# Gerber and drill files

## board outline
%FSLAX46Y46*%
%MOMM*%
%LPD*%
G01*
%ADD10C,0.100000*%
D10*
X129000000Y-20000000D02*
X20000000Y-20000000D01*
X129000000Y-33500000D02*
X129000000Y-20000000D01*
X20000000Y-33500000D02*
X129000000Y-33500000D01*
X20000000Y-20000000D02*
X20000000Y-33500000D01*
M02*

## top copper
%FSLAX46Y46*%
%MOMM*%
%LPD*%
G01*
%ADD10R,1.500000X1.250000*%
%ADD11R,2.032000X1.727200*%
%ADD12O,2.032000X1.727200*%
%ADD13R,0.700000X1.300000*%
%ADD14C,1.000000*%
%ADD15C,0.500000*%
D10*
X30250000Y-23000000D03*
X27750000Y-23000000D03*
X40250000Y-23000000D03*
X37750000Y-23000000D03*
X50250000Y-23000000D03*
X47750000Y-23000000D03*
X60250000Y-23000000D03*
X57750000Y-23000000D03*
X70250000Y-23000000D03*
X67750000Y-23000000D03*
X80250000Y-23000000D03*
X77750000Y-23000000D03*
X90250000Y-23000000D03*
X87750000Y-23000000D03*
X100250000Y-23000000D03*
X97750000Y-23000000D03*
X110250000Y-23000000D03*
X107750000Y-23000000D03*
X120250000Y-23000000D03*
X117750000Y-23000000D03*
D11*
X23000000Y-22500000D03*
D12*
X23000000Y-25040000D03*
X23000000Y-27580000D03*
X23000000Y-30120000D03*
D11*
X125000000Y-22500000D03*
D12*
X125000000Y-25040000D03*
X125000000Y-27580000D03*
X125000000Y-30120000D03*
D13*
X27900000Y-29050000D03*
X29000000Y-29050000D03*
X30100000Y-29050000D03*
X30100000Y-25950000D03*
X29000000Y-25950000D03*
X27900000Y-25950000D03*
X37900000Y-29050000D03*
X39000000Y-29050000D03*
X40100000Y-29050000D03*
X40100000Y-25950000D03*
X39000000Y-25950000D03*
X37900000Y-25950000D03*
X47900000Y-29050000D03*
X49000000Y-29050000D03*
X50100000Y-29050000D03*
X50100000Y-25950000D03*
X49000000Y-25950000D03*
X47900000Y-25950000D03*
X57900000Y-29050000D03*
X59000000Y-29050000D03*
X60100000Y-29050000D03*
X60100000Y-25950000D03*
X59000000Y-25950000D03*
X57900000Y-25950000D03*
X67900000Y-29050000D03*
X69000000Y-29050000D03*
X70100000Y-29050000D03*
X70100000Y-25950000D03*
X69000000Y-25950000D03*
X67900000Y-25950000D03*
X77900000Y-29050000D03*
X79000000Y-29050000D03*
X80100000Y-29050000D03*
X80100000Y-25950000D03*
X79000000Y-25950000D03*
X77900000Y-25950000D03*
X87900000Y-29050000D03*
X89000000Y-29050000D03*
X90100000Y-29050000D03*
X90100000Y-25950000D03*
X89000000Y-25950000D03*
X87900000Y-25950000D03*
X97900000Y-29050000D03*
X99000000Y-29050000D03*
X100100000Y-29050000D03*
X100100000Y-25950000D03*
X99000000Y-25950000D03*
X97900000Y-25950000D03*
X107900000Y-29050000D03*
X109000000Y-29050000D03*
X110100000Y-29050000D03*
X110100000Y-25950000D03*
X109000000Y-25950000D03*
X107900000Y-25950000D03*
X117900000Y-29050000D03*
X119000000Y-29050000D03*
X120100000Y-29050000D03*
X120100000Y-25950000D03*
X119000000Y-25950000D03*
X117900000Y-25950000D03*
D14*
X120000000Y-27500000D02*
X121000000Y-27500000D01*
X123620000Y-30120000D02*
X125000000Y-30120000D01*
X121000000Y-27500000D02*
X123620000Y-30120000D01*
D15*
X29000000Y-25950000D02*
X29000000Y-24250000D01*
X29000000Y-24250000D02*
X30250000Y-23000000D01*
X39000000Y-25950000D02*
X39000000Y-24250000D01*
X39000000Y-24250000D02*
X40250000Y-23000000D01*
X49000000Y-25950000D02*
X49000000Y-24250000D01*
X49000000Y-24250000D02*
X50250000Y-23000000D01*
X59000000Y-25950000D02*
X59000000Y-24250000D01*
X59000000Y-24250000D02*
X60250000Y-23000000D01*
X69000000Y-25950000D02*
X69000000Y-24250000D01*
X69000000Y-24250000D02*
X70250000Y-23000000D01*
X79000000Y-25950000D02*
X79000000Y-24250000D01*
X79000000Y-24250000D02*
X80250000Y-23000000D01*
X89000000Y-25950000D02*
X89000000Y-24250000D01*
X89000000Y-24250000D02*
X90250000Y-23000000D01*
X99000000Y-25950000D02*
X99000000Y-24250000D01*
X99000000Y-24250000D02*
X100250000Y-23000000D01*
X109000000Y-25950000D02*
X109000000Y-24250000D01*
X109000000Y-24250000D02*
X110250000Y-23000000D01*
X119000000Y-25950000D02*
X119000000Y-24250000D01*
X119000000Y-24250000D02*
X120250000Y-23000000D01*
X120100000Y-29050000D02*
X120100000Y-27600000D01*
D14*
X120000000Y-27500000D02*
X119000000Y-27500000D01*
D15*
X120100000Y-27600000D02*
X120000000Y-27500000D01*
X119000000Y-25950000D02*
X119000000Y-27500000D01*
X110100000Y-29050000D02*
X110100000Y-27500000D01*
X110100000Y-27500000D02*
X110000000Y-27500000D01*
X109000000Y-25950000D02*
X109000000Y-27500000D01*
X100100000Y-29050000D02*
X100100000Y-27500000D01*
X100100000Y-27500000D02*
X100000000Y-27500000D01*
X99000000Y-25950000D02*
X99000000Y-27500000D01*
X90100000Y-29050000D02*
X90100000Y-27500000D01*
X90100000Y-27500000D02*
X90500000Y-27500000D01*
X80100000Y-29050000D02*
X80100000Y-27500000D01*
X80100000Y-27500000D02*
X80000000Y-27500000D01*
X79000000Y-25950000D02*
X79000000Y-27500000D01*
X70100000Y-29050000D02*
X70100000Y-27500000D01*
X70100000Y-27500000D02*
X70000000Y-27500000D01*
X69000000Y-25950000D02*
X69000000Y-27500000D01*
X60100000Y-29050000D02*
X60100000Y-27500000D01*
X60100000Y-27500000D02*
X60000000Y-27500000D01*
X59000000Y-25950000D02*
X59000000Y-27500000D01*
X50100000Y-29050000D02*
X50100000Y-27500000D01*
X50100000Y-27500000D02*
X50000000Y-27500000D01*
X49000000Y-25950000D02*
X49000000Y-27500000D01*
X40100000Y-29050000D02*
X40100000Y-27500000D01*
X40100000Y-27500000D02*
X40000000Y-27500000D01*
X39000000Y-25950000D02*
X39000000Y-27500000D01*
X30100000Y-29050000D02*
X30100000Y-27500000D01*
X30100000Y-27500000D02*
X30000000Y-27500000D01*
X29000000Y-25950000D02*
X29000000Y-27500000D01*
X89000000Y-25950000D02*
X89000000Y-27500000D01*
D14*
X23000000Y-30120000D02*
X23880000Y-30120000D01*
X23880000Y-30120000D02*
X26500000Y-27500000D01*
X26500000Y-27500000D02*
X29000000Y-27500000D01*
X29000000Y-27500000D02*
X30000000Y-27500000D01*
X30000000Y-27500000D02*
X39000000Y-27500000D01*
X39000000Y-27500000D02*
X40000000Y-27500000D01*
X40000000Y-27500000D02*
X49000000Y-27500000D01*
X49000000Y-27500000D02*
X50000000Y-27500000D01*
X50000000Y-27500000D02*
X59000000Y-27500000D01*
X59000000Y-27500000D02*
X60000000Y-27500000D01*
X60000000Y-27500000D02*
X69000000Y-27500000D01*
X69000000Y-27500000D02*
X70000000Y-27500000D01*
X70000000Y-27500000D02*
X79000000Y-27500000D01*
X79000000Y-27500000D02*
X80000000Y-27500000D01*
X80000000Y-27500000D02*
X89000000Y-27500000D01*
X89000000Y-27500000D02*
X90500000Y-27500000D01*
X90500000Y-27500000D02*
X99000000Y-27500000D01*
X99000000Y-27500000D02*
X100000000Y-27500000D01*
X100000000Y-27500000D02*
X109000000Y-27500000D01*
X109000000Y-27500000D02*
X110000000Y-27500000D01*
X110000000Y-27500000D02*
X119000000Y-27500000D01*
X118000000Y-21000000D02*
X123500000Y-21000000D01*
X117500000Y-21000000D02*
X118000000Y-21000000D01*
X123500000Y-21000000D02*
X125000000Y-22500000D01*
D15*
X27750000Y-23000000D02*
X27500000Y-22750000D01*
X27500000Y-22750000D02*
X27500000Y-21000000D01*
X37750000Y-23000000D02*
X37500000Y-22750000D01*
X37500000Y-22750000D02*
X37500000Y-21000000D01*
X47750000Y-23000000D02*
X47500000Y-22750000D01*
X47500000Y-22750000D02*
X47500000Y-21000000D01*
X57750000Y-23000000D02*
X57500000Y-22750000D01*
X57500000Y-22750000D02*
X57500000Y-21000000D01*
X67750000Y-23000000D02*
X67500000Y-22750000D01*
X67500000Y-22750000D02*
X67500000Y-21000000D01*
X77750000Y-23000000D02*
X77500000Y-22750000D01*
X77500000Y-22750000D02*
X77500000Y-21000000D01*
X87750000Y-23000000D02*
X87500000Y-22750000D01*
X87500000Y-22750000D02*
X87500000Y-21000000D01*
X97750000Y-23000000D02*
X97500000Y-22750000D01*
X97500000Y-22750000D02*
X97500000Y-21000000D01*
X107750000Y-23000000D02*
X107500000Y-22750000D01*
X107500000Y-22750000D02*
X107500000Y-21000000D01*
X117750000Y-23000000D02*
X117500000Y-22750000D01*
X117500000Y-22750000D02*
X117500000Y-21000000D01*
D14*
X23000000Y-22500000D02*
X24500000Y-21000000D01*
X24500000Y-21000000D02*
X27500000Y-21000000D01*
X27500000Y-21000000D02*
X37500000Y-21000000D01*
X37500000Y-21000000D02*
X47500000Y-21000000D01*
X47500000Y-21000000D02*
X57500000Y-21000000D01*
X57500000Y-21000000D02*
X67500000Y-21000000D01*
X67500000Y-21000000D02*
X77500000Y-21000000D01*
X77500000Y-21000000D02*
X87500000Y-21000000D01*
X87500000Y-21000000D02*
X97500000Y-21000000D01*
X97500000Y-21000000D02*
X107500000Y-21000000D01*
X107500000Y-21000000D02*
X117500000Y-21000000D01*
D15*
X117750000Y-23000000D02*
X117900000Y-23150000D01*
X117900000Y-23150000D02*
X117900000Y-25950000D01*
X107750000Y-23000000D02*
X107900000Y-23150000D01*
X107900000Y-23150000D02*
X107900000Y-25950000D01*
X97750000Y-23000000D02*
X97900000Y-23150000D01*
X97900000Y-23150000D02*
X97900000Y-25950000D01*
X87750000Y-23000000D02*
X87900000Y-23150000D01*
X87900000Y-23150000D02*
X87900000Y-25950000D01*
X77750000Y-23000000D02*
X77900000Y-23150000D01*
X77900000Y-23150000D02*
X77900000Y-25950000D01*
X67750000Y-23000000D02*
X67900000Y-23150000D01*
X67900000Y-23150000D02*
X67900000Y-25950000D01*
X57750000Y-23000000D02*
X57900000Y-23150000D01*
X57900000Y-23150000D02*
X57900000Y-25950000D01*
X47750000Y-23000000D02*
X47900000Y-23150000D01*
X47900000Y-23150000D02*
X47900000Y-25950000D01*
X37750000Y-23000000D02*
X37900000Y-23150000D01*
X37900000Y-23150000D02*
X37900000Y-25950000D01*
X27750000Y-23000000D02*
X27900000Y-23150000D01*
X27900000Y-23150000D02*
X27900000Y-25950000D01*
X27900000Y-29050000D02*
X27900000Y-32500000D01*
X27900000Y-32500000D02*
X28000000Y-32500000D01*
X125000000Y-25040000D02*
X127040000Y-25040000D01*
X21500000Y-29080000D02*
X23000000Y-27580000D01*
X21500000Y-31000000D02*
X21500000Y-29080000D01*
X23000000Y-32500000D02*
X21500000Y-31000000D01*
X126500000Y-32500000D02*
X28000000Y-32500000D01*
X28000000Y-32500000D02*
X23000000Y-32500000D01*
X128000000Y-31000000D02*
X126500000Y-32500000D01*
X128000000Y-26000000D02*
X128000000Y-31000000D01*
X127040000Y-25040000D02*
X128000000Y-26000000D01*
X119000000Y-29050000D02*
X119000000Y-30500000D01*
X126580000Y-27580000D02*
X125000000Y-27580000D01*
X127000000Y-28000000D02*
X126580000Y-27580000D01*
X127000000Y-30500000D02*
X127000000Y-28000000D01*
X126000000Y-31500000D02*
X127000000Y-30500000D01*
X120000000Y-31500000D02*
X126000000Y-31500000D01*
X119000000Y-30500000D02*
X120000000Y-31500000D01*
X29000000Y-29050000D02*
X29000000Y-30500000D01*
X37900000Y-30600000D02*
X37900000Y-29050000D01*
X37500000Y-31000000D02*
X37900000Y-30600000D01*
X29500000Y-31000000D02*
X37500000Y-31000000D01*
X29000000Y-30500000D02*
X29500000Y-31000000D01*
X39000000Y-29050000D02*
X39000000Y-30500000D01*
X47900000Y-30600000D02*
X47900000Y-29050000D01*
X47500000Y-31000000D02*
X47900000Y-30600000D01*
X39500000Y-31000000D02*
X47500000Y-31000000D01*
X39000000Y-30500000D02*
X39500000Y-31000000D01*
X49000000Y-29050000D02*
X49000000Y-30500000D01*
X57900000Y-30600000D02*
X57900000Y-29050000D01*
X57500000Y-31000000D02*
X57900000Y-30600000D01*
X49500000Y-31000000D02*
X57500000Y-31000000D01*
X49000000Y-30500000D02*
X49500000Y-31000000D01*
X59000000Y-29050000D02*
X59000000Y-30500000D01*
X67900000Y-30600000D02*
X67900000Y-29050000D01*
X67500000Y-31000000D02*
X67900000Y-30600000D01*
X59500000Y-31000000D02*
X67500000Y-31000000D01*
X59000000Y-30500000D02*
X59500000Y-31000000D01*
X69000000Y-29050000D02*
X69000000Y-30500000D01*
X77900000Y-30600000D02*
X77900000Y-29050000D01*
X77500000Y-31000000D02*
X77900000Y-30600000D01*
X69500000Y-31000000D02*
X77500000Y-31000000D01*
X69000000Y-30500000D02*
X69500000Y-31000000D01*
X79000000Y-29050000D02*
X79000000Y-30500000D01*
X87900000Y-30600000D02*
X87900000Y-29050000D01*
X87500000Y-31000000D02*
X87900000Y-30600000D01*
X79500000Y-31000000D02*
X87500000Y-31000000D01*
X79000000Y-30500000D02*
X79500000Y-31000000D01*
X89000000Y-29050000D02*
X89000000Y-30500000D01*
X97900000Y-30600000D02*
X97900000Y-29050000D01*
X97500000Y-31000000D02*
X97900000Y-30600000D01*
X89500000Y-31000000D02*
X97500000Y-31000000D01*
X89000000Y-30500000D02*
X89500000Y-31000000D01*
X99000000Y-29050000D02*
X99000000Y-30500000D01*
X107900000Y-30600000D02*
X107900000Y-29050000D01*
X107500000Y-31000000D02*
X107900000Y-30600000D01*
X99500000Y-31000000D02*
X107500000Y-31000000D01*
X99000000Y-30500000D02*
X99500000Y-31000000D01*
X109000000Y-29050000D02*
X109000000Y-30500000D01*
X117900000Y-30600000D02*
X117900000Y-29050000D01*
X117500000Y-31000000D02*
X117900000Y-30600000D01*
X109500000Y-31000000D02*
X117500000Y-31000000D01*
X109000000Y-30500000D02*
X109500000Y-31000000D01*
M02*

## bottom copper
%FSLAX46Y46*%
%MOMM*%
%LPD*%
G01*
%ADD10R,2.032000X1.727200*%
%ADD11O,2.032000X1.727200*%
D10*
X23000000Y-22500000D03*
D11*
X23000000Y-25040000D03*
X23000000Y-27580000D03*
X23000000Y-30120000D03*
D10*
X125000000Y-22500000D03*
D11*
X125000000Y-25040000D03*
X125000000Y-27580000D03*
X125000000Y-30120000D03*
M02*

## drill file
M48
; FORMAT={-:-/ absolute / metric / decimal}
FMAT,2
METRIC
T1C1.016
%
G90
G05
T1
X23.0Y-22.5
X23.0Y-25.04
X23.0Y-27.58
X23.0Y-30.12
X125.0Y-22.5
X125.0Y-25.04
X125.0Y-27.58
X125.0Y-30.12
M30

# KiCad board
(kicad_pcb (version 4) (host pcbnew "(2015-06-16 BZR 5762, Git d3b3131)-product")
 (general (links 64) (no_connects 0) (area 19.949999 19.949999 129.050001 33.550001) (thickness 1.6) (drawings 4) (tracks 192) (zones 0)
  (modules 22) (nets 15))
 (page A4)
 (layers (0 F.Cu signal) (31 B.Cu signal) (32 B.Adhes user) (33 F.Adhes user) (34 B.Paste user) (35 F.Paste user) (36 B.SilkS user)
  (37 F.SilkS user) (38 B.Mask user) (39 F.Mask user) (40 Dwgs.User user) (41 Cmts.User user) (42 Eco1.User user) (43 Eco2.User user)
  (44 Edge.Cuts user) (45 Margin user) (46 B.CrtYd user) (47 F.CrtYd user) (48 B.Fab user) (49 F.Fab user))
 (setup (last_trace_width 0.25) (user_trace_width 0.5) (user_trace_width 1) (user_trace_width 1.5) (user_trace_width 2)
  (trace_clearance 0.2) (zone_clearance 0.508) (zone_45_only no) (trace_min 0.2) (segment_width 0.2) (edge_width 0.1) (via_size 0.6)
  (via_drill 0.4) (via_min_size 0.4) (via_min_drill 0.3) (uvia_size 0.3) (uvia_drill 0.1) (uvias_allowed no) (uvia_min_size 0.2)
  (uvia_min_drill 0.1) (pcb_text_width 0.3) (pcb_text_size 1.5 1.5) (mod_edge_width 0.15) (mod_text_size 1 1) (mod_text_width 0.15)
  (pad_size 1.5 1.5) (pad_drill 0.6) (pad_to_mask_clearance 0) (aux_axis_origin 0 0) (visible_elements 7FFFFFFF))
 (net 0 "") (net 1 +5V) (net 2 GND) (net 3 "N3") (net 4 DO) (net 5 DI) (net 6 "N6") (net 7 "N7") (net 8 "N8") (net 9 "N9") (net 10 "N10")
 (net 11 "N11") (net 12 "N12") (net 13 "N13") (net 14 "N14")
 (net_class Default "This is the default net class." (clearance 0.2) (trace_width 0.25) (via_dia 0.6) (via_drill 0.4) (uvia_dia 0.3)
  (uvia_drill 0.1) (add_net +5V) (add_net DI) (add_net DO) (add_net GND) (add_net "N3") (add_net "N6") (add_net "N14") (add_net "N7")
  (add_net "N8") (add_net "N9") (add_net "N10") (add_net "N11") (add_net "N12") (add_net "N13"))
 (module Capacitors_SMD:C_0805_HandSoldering (layer F.Cu) (at 29 23 180)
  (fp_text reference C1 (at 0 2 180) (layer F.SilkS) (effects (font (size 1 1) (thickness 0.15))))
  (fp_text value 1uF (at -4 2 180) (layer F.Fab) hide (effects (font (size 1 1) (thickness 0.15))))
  (pad 1 smd rect (at -1.25 0 180) (size 1.5 1.25) (layers F.Cu F.Paste F.Mask) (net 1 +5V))
  (pad 2 smd rect (at 1.25 0 180) (size 1.5 1.25) (layers F.Cu F.Paste F.Mask) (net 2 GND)))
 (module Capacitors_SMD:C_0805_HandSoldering (layer F.Cu) (at 39 23 180)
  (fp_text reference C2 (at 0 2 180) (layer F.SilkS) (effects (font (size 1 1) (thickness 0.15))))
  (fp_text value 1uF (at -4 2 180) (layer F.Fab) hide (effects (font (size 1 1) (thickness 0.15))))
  (pad 1 smd rect (at -1.25 0 180) (size 1.5 1.25) (layers F.Cu F.Paste F.Mask) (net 1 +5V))
  (pad 2 smd rect (at 1.25 0 180) (size 1.5 1.25) (layers F.Cu F.Paste F.Mask) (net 2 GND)))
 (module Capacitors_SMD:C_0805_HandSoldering (layer F.Cu) (at 49 23 180)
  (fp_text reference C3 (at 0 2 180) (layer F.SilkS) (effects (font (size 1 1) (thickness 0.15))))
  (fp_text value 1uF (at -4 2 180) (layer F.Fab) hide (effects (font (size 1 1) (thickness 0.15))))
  (pad 1 smd rect (at -1.25 0 180) (size 1.5 1.25) (layers F.Cu F.Paste F.Mask) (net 1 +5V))
  (pad 2 smd rect (at 1.25 0 180) (size 1.5 1.25) (layers F.Cu F.Paste F.Mask) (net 2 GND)))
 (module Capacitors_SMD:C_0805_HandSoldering (layer F.Cu) (at 59 23 180)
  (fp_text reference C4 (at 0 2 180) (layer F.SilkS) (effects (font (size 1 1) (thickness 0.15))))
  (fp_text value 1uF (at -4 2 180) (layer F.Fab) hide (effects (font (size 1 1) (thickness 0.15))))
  (pad 1 smd rect (at -1.25 0 180) (size 1.5 1.25) (layers F.Cu F.Paste F.Mask) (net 1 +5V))
  (pad 2 smd rect (at 1.25 0 180) (size 1.5 1.25) (layers F.Cu F.Paste F.Mask) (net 2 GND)))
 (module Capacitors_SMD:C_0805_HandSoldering (layer F.Cu) (at 69 23 180)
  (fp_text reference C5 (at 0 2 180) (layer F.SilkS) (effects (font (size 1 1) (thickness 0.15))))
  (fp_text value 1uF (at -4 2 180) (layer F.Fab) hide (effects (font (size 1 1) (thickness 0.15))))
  (pad 1 smd rect (at -1.25 0 180) (size 1.5 1.25) (layers F.Cu F.Paste F.Mask) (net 1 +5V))
  (pad 2 smd rect (at 1.25 0 180) (size 1.5 1.25) (layers F.Cu F.Paste F.Mask) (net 2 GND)))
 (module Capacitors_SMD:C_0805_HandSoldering (layer F.Cu) (at 79 23 180)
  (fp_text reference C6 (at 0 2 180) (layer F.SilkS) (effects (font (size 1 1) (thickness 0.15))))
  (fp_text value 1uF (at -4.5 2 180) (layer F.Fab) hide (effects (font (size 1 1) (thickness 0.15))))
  (pad 1 smd rect (at -1.25 0 180) (size 1.5 1.25) (layers F.Cu F.Paste F.Mask) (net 1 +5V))
  (pad 2 smd rect (at 1.25 0 180) (size 1.5 1.25) (layers F.Cu F.Paste F.Mask) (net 2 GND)))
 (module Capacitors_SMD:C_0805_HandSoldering (layer F.Cu) (at 89 23 180)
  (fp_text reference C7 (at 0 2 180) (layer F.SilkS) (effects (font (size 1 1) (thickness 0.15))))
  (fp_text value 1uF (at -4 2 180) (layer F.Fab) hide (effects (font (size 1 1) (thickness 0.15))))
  (pad 1 smd rect (at -1.25 0 180) (size 1.5 1.25) (layers F.Cu F.Paste F.Mask) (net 1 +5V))
  (pad 2 smd rect (at 1.25 0 180) (size 1.5 1.25) (layers F.Cu F.Paste F.Mask) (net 2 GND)))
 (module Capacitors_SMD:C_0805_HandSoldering (layer F.Cu) (at 99 23 180)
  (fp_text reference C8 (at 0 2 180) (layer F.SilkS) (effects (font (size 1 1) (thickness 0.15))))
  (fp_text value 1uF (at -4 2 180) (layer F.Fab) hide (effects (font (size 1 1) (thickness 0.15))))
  (pad 1 smd rect (at -1.25 0 180) (size 1.5 1.25) (layers F.Cu F.Paste F.Mask) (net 1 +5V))
  (pad 2 smd rect (at 1.25 0 180) (size 1.5 1.25) (layers F.Cu F.Paste F.Mask) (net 2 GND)))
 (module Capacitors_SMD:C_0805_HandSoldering (layer F.Cu) (at 109 23 180)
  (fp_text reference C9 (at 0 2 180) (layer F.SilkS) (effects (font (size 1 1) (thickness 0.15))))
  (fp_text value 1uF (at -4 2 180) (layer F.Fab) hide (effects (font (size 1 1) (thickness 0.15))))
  (pad 1 smd rect (at -1.25 0 180) (size 1.5 1.25) (layers F.Cu F.Paste F.Mask) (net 1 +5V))
  (pad 2 smd rect (at 1.25 0 180) (size 1.5 1.25) (layers F.Cu F.Paste F.Mask) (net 2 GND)))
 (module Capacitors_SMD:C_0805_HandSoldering (layer F.Cu) (at 119 23 180)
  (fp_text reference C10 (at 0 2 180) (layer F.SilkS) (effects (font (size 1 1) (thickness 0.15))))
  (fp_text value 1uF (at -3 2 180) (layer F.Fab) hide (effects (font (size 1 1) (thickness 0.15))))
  (pad 1 smd rect (at -1.25 0 180) (size 1.5 1.25) (layers F.Cu F.Paste F.Mask) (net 1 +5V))
  (pad 2 smd rect (at 1.25 0 180) (size 1.5 1.25) (layers F.Cu F.Paste F.Mask) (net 2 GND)))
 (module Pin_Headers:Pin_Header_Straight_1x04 (layer F.Cu) (at 23 22.5)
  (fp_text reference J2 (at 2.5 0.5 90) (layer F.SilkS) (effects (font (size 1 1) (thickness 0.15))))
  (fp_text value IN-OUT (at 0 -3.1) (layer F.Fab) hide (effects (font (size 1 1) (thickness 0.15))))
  (pad 1 thru_hole rect (at 0 0) (size 2.032 1.7272) (drill 1.016) (layers *.Cu *.Mask F.SilkS) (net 2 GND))
  (pad 2 thru_hole oval (at 0 2.54) (size 2.032 1.7272) (drill 1.016) (layers *.Cu *.Mask F.SilkS) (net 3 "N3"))
  (pad 3 thru_hole oval (at 0 5.08) (size 2.032 1.7272) (drill 1.016) (layers *.Cu *.Mask F.SilkS) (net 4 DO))
  (pad 4 thru_hole oval (at 0 7.62) (size 2.032 1.7272) (drill 1.016) (layers *.Cu *.Mask F.SilkS) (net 1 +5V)))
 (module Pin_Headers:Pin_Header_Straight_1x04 (layer F.Cu) (at 125 22.5)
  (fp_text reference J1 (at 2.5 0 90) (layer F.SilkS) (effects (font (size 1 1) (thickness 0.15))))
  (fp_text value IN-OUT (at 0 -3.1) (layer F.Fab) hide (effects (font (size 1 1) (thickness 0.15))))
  (pad 1 thru_hole rect (at 0 0) (size 2.032 1.7272) (drill 1.016) (layers *.Cu *.Mask F.SilkS) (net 2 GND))
  (pad 2 thru_hole oval (at 0 2.54) (size 2.032 1.7272) (drill 1.016) (layers *.Cu *.Mask F.SilkS) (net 4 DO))
  (pad 3 thru_hole oval (at 0 5.08) (size 2.032 1.7272) (drill 1.016) (layers *.Cu *.Mask F.SilkS) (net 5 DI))
  (pad 4 thru_hole oval (at 0 7.62) (size 2.032 1.7272) (drill 1.016) (layers *.Cu *.Mask F.SilkS) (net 1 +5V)))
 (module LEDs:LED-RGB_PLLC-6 (layer F.Cu) (at 29 27.5 90)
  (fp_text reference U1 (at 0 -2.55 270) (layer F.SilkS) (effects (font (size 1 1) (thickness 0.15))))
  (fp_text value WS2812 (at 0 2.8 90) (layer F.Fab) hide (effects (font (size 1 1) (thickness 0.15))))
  (pad 1 smd rect (at -1.55 -1.1 180) (size 0.7 1.3) (layers F.Cu F.Paste F.Mask) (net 4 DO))
  (pad 2 smd rect (at -1.55 0 180) (size 0.7 1.3) (layers F.Cu F.Paste F.Mask) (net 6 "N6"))
  (pad 3 smd rect (at -1.55 1.1 180) (size 0.7 1.3) (layers F.Cu F.Paste F.Mask) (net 1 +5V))
  (pad 4 smd rect (at 1.55 1.1 180) (size 0.7 1.3) (layers F.Cu F.Paste F.Mask))
  (pad 5 smd rect (at 1.55 0 180) (size 0.7 1.3) (layers F.Cu F.Paste F.Mask) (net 1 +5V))
  (pad 6 smd rect (at 1.55 -1.1 180) (size 0.7 1.3) (layers F.Cu F.Paste F.Mask) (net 2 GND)))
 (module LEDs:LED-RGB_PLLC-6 (layer F.Cu) (at 39 27.5 90)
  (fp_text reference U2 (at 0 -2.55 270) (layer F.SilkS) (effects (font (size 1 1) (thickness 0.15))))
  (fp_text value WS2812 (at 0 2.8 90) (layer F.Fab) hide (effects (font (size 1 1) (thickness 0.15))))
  (pad 1 smd rect (at -1.55 -1.1 180) (size 0.7 1.3) (layers F.Cu F.Paste F.Mask) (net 6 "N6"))
  (pad 2 smd rect (at -1.55 0 180) (size 0.7 1.3) (layers F.Cu F.Paste F.Mask) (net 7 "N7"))
  (pad 3 smd rect (at -1.55 1.1 180) (size 0.7 1.3) (layers F.Cu F.Paste F.Mask) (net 1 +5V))
  (pad 4 smd rect (at 1.55 1.1 180) (size 0.7 1.3) (layers F.Cu F.Paste F.Mask))
  (pad 5 smd rect (at 1.55 0 180) (size 0.7 1.3) (layers F.Cu F.Paste F.Mask) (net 1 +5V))
  (pad 6 smd rect (at 1.55 -1.1 180) (size 0.7 1.3) (layers F.Cu F.Paste F.Mask) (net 2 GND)))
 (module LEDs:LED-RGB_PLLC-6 (layer F.Cu) (at 49 27.5 90)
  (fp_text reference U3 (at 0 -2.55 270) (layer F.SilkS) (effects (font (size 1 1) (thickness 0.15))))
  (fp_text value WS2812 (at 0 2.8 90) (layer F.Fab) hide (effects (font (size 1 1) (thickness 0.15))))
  (pad 1 smd rect (at -1.55 -1.1 180) (size 0.7 1.3) (layers F.Cu F.Paste F.Mask) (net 7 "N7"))
  (pad 2 smd rect (at -1.55 0 180) (size 0.7 1.3) (layers F.Cu F.Paste F.Mask) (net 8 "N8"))
  (pad 3 smd rect (at -1.55 1.1 180) (size 0.7 1.3) (layers F.Cu F.Paste F.Mask) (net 1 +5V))
  (pad 4 smd rect (at 1.55 1.1 180) (size 0.7 1.3) (layers F.Cu F.Paste F.Mask))
  (pad 5 smd rect (at 1.55 0 180) (size 0.7 1.3) (layers F.Cu F.Paste F.Mask) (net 1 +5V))
  (pad 6 smd rect (at 1.55 -1.1 180) (size 0.7 1.3) (layers F.Cu F.Paste F.Mask) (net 2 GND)))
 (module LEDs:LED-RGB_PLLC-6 (layer F.Cu) (at 59 27.5 90)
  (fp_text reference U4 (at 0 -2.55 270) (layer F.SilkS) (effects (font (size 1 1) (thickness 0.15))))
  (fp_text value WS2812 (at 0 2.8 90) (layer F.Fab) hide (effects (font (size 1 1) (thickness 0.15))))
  (pad 1 smd rect (at -1.55 -1.1 180) (size 0.7 1.3) (layers F.Cu F.Paste F.Mask) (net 8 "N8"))
  (pad 2 smd rect (at -1.55 0 180) (size 0.7 1.3) (layers F.Cu F.Paste F.Mask) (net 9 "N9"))
  (pad 3 smd rect (at -1.55 1.1 180) (size 0.7 1.3) (layers F.Cu F.Paste F.Mask) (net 1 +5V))
  (pad 4 smd rect (at 1.55 1.1 180) (size 0.7 1.3) (layers F.Cu F.Paste F.Mask))
  (pad 5 smd rect (at 1.55 0 180) (size 0.7 1.3) (layers F.Cu F.Paste F.Mask) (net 1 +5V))
  (pad 6 smd rect (at 1.55 -1.1 180) (size 0.7 1.3) (layers F.Cu F.Paste F.Mask) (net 2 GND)))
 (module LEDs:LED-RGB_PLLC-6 (layer F.Cu) (at 69 27.5 90)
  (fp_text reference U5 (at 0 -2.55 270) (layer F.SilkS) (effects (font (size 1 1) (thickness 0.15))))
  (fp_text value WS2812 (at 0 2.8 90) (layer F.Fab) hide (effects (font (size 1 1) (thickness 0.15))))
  (pad 1 smd rect (at -1.55 -1.1 180) (size 0.7 1.3) (layers F.Cu F.Paste F.Mask) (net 9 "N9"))
  (pad 2 smd rect (at -1.55 0 180) (size 0.7 1.3) (layers F.Cu F.Paste F.Mask) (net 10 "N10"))
  (pad 3 smd rect (at -1.55 1.1 180) (size 0.7 1.3) (layers F.Cu F.Paste F.Mask) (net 1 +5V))
  (pad 4 smd rect (at 1.55 1.1 180) (size 0.7 1.3) (layers F.Cu F.Paste F.Mask))
  (pad 5 smd rect (at 1.55 0 180) (size 0.7 1.3) (layers F.Cu F.Paste F.Mask) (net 1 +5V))
  (pad 6 smd rect (at 1.55 -1.1 180) (size 0.7 1.3) (layers F.Cu F.Paste F.Mask) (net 2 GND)))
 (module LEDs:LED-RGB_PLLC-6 (layer F.Cu) (at 79 27.5 90)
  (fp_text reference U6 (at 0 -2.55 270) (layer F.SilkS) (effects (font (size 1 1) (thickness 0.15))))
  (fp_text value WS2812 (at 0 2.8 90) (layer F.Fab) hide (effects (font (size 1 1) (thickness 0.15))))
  (pad 1 smd rect (at -1.55 -1.1 180) (size 0.7 1.3) (layers F.Cu F.Paste F.Mask) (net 10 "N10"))
  (pad 2 smd rect (at -1.55 0 180) (size 0.7 1.3) (layers F.Cu F.Paste F.Mask) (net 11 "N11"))
  (pad 3 smd rect (at -1.55 1.1 180) (size 0.7 1.3) (layers F.Cu F.Paste F.Mask) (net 1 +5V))
  (pad 4 smd rect (at 1.55 1.1 180) (size 0.7 1.3) (layers F.Cu F.Paste F.Mask))
  (pad 5 smd rect (at 1.55 0 180) (size 0.7 1.3) (layers F.Cu F.Paste F.Mask) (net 1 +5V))
  (pad 6 smd rect (at 1.55 -1.1 180) (size 0.7 1.3) (layers F.Cu F.Paste F.Mask) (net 2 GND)))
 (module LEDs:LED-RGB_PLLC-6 (layer F.Cu) (at 89 27.5 90)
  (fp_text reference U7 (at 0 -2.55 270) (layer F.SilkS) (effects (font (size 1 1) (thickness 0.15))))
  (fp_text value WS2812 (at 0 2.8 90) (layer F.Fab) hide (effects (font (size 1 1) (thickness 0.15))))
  (pad 1 smd rect (at -1.55 -1.1 180) (size 0.7 1.3) (layers F.Cu F.Paste F.Mask) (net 11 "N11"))
  (pad 2 smd rect (at -1.55 0 180) (size 0.7 1.3) (layers F.Cu F.Paste F.Mask) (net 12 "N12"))
  (pad 3 smd rect (at -1.55 1.1 180) (size 0.7 1.3) (layers F.Cu F.Paste F.Mask) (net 1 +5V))
  (pad 4 smd rect (at 1.55 1.1 180) (size 0.7 1.3) (layers F.Cu F.Paste F.Mask))
  (pad 5 smd rect (at 1.55 0 180) (size 0.7 1.3) (layers F.Cu F.Paste F.Mask) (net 1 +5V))
  (pad 6 smd rect (at 1.55 -1.1 180) (size 0.7 1.3) (layers F.Cu F.Paste F.Mask) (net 2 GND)))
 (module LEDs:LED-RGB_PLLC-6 (layer F.Cu) (at 99 27.5 90)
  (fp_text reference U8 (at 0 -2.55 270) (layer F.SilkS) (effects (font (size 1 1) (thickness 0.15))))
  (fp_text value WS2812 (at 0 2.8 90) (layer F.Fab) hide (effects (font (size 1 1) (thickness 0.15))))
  (pad 1 smd rect (at -1.55 -1.1 180) (size 0.7 1.3) (layers F.Cu F.Paste F.Mask) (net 12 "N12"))
  (pad 2 smd rect (at -1.55 0 180) (size 0.7 1.3) (layers F.Cu F.Paste F.Mask) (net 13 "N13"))
  (pad 3 smd rect (at -1.55 1.1 180) (size 0.7 1.3) (layers F.Cu F.Paste F.Mask) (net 1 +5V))
  (pad 4 smd rect (at 1.55 1.1 180) (size 0.7 1.3) (layers F.Cu F.Paste F.Mask))
  (pad 5 smd rect (at 1.55 0 180) (size 0.7 1.3) (layers F.Cu F.Paste F.Mask) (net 1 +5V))
  (pad 6 smd rect (at 1.55 -1.1 180) (size 0.7 1.3) (layers F.Cu F.Paste F.Mask) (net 2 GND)))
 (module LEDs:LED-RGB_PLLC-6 (layer F.Cu) (at 109 27.5 90)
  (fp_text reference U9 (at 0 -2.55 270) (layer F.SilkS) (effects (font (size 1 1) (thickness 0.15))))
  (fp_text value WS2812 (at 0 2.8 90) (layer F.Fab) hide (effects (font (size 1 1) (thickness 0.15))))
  (pad 1 smd rect (at -1.55 -1.1 180) (size 0.7 1.3) (layers F.Cu F.Paste F.Mask) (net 13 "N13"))
  (pad 2 smd rect (at -1.55 0 180) (size 0.7 1.3) (layers F.Cu F.Paste F.Mask) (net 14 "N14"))
  (pad 3 smd rect (at -1.55 1.1 180) (size 0.7 1.3) (layers F.Cu F.Paste F.Mask) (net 1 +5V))
  (pad 4 smd rect (at 1.55 1.1 180) (size 0.7 1.3) (layers F.Cu F.Paste F.Mask))
  (pad 5 smd rect (at 1.55 0 180) (size 0.7 1.3) (layers F.Cu F.Paste F.Mask) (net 1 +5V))
  (pad 6 smd rect (at 1.55 -1.1 180) (size 0.7 1.3) (layers F.Cu F.Paste F.Mask) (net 2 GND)))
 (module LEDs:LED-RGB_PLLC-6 (layer F.Cu) (at 119 27.5 90)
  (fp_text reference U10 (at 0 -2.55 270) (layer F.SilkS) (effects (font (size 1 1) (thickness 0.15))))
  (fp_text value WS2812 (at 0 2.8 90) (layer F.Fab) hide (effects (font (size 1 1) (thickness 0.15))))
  (pad 1 smd rect (at -1.55 -1.1 180) (size 0.7 1.3) (layers F.Cu F.Paste F.Mask) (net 14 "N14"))
  (pad 2 smd rect (at -1.55 0 180) (size 0.7 1.3) (layers F.Cu F.Paste F.Mask) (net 5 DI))
  (pad 3 smd rect (at -1.55 1.1 180) (size 0.7 1.3) (layers F.Cu F.Paste F.Mask) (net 1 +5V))
  (pad 4 smd rect (at 1.55 1.1 180) (size 0.7 1.3) (layers F.Cu F.Paste F.Mask))
  (pad 5 smd rect (at 1.55 0 180) (size 0.7 1.3) (layers F.Cu F.Paste F.Mask) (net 1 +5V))
  (pad 6 smd rect (at 1.55 -1.1 180) (size 0.7 1.3) (layers F.Cu F.Paste F.Mask) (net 2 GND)))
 (gr_line (start 129 20) (end 20 20) (angle 90) (layer Edge.Cuts) (width 0.1))
 (gr_line (start 129 33.5) (end 129 20) (angle 90) (layer Edge.Cuts) (width 0.1))
 (gr_line (start 20 33.5) (end 129 33.5) (angle 90) (layer Edge.Cuts) (width 0.1))
 (gr_line (start 20 20) (end 20 33.5) (angle 90) (layer Edge.Cuts) (width 0.1))
 (segment (start 120 27.5) (end 121 27.5) (width 1) (layer F.Cu) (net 1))
 (segment (start 123.62 30.12) (end 125 30.12) (width 1) (layer F.Cu) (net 1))
 (segment (start 121 27.5) (end 123.62 30.12) (width 1) (layer F.Cu) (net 1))
 (segment (start 29 25.95) (end 29 24.25) (width 0.5) (layer F.Cu) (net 1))
 (segment (start 29 24.25) (end 30.25 23) (width 0.5) (layer F.Cu) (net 1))
 (segment (start 39 25.95) (end 39 24.25) (width 0.5) (layer F.Cu) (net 1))
 (segment (start 39 24.25) (end 40.25 23) (width 0.5) (layer F.Cu) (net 1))
 (segment (start 49 25.95) (end 49 24.25) (width 0.5) (layer F.Cu) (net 1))
 (segment (start 49 24.25) (end 50.25 23) (width 0.5) (layer F.Cu) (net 1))
 (segment (start 59 25.95) (end 59 24.25) (width 0.5) (layer F.Cu) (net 1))
 (segment (start 59 24.25) (end 60.25 23) (width 0.5) (layer F.Cu) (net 1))
 (segment (start 69 25.95) (end 69 24.25) (width 0.5) (layer F.Cu) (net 1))
 (segment (start 69 24.25) (end 70.25 23) (width 0.5) (layer F.Cu) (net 1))
 (segment (start 79 25.95) (end 79 24.25) (width 0.5) (layer F.Cu) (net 1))
 (segment (start 79 24.25) (end 80.25 23) (width 0.5) (layer F.Cu) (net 1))
 (segment (start 89 25.95) (end 89 24.25) (width 0.5) (layer F.Cu) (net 1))
 (segment (start 89 24.25) (end 90.25 23) (width 0.5) (layer F.Cu) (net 1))
 (segment (start 99 25.95) (end 99 24.25) (width 0.5) (layer F.Cu) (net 1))
 (segment (start 99 24.25) (end 100.25 23) (width 0.5) (layer F.Cu) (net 1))
 (segment (start 109 25.95) (end 109 24.25) (width 0.5) (layer F.Cu) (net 1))
 (segment (start 109 24.25) (end 110.25 23) (width 0.5) (layer F.Cu) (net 1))
 (segment (start 119 25.95) (end 119 24.25) (width 0.5) (layer F.Cu) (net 1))
 (segment (start 119 24.25) (end 120.25 23) (width 0.5) (layer F.Cu) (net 1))
 (segment (start 120.1 29.05) (end 120.1 27.6) (width 0.5) (layer F.Cu) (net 1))
 (segment (start 120 27.5) (end 119 27.5) (width 1) (layer F.Cu) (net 1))
 (segment (start 120.1 27.6) (end 120 27.5) (width 0.5) (layer F.Cu) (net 1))
 (segment (start 119 25.95) (end 119 27.5) (width 0.5) (layer F.Cu) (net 1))
 (segment (start 110.1 29.05) (end 110.1 27.5) (width 0.5) (layer F.Cu) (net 1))
 (segment (start 110.1 27.5) (end 110 27.5) (width 0.5) (layer F.Cu) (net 1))
 (segment (start 109 25.95) (end 109 27.5) (width 0.5) (layer F.Cu) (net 1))
 (segment (start 100.1 29.05) (end 100.1 27.5) (width 0.5) (layer F.Cu) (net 1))
 (segment (start 100.1 27.5) (end 100 27.5) (width 0.5) (layer F.Cu) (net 1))
 (segment (start 99 25.95) (end 99 27.5) (width 0.5) (layer F.Cu) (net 1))
 (segment (start 90.1 29.05) (end 90.1 27.5) (width 0.5) (layer F.Cu) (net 1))
 (segment (start 90.1 27.5) (end 90.5 27.5) (width 0.5) (layer F.Cu) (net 1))
 (segment (start 80.1 29.05) (end 80.1 27.5) (width 0.5) (layer F.Cu) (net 1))
 (segment (start 80.1 27.5) (end 80 27.5) (width 0.5) (layer F.Cu) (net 1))
 (segment (start 79 25.95) (end 79 27.5) (width 0.5) (layer F.Cu) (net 1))
 (segment (start 70.1 29.05) (end 70.1 27.5) (width 0.5) (layer F.Cu) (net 1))
 (segment (start 70.1 27.5) (end 70 27.5) (width 0.5) (layer F.Cu) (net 1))
 (segment (start 69 25.95) (end 69 27.5) (width 0.5) (layer F.Cu) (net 1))
 (segment (start 60.1 29.05) (end 60.1 27.5) (width 0.5) (layer F.Cu) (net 1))
 (segment (start 60.1 27.5) (end 60 27.5) (width 0.5) (layer F.Cu) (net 1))
 (segment (start 59 25.95) (end 59 27.5) (width 0.5) (layer F.Cu) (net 1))
 (segment (start 50.1 29.05) (end 50.1 27.5) (width 0.5) (layer F.Cu) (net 1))
 (segment (start 50.1 27.5) (end 50 27.5) (width 0.5) (layer F.Cu) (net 1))
 (segment (start 49 25.95) (end 49 27.5) (width 0.5) (layer F.Cu) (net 1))
 (segment (start 40.1 29.05) (end 40.1 27.5) (width 0.5) (layer F.Cu) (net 1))
 (segment (start 40.1 27.5) (end 40 27.5) (width 0.5) (layer F.Cu) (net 1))
 (segment (start 39 25.95) (end 39 27.5) (width 0.5) (layer F.Cu) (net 1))
 (segment (start 30.1 29.05) (end 30.1 27.5) (width 0.5) (layer F.Cu) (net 1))
 (segment (start 30.1 27.5) (end 30 27.5) (width 0.5) (layer F.Cu) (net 1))
 (segment (start 29 25.95) (end 29 27.5) (width 0.5) (layer F.Cu) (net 1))
 (segment (start 89 25.95) (end 89 27.5) (width 0.5) (layer F.Cu) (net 1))
 (segment (start 23 30.12) (end 23.88 30.12) (width 1) (layer F.Cu) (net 1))
 (segment (start 23.88 30.12) (end 26.5 27.5) (width 1) (layer F.Cu) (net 1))
 (segment (start 26.5 27.5) (end 29 27.5) (width 1) (layer F.Cu) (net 1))
 (segment (start 29 27.5) (end 30 27.5) (width 1) (layer F.Cu) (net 1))
 (segment (start 30 27.5) (end 39 27.5) (width 1) (layer F.Cu) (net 1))
 (segment (start 39 27.5) (end 40 27.5) (width 1) (layer F.Cu) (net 1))
 (segment (start 40 27.5) (end 49 27.5) (width 1) (layer F.Cu) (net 1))
 (segment (start 49 27.5) (end 50 27.5) (width 1) (layer F.Cu) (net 1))
 (segment (start 50 27.5) (end 59 27.5) (width 1) (layer F.Cu) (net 1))
 (segment (start 59 27.5) (end 60 27.5) (width 1) (layer F.Cu) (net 1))
 (segment (start 60 27.5) (end 69 27.5) (width 1) (layer F.Cu) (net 1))
 (segment (start 69 27.5) (end 70 27.5) (width 1) (layer F.Cu) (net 1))
 (segment (start 70 27.5) (end 79 27.5) (width 1) (layer F.Cu) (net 1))
 (segment (start 79 27.5) (end 80 27.5) (width 1) (layer F.Cu) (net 1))
 (segment (start 80 27.5) (end 89 27.5) (width 1) (layer F.Cu) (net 1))
 (segment (start 89 27.5) (end 90.5 27.5) (width 1) (layer F.Cu) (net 1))
 (segment (start 90.5 27.5) (end 99 27.5) (width 1) (layer F.Cu) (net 1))
 (segment (start 99 27.5) (end 100 27.5) (width 1) (layer F.Cu) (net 1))
 (segment (start 100 27.5) (end 109 27.5) (width 1) (layer F.Cu) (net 1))
 (segment (start 109 27.5) (end 110 27.5) (width 1) (layer F.Cu) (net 1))
 (segment (start 110 27.5) (end 119 27.5) (width 1) (layer F.Cu) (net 1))
 (segment (start 118 21) (end 123.5 21) (width 1) (layer F.Cu) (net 2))
 (segment (start 117.5 21) (end 118 21) (width 1) (layer F.Cu) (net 2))
 (segment (start 123.5 21) (end 125 22.5) (width 1) (layer F.Cu) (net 2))
 (segment (start 27.75 23) (end 27.5 22.75) (width 0.5) (layer F.Cu) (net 2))
 (segment (start 27.5 22.75) (end 27.5 21) (width 0.5) (layer F.Cu) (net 2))
 (segment (start 37.75 23) (end 37.5 22.75) (width 0.5) (layer F.Cu) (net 2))
 (segment (start 37.5 22.75) (end 37.5 21) (width 0.5) (layer F.Cu) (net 2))
 (segment (start 47.75 23) (end 47.5 22.75) (width 0.5) (layer F.Cu) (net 2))
 (segment (start 47.5 22.75) (end 47.5 21) (width 0.5) (layer F.Cu) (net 2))
 (segment (start 57.75 23) (end 57.5 22.75) (width 0.5) (layer F.Cu) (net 2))
 (segment (start 57.5 22.75) (end 57.5 21) (width 0.5) (layer F.Cu) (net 2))
 (segment (start 67.75 23) (end 67.5 22.75) (width 0.5) (layer F.Cu) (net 2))
 (segment (start 67.5 22.75) (end 67.5 21) (width 0.5) (layer F.Cu) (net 2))
 (segment (start 77.75 23) (end 77.5 22.75) (width 0.5) (layer F.Cu) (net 2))
 (segment (start 77.5 22.75) (end 77.5 21) (width 0.5) (layer F.Cu) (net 2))
 (segment (start 87.75 23) (end 87.5 22.75) (width 0.5) (layer F.Cu) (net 2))
 (segment (start 87.5 22.75) (end 87.5 21) (width 0.5) (layer F.Cu) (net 2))
 (segment (start 97.75 23) (end 97.5 22.75) (width 0.5) (layer F.Cu) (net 2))
 (segment (start 97.5 22.75) (end 97.5 21) (width 0.5) (layer F.Cu) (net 2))
 (segment (start 107.75 23) (end 107.5 22.75) (width 0.5) (layer F.Cu) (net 2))
 (segment (start 107.5 22.75) (end 107.5 21) (width 0.5) (layer F.Cu) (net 2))
 (segment (start 117.75 23) (end 117.5 22.75) (width 0.5) (layer F.Cu) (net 2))
 (segment (start 117.5 22.75) (end 117.5 21) (width 0.5) (layer F.Cu) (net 2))
 (segment (start 23 22.5) (end 24.5 21) (width 1) (layer F.Cu) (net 2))
 (segment (start 24.5 21) (end 27.5 21) (width 1) (layer F.Cu) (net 2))
 (segment (start 27.5 21) (end 37.5 21) (width 1) (layer F.Cu) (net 2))
 (segment (start 37.5 21) (end 47.5 21) (width 1) (layer F.Cu) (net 2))
 (segment (start 47.5 21) (end 57.5 21) (width 1) (layer F.Cu) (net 2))
 (segment (start 57.5 21) (end 67.5 21) (width 1) (layer F.Cu) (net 2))
 (segment (start 67.5 21) (end 77.5 21) (width 1) (layer F.Cu) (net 2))
 (segment (start 77.5 21) (end 87.5 21) (width 1) (layer F.Cu) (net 2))
 (segment (start 87.5 21) (end 97.5 21) (width 1) (layer F.Cu) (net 2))
 (segment (start 97.5 21) (end 107.5 21) (width 1) (layer F.Cu) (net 2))
 (segment (start 107.5 21) (end 117.5 21) (width 1) (layer F.Cu) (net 2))
 (segment (start 117.75 23) (end 117.9 23.15) (width 0.5) (layer F.Cu) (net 2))
 (segment (start 117.9 23.15) (end 117.9 25.95) (width 0.5) (layer F.Cu) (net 2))
 (segment (start 107.75 23) (end 107.9 23.15) (width 0.5) (layer F.Cu) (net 2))
 (segment (start 107.9 23.15) (end 107.9 25.95) (width 0.5) (layer F.Cu) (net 2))
 (segment (start 97.75 23) (end 97.9 23.15) (width 0.5) (layer F.Cu) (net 2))
 (segment (start 97.9 23.15) (end 97.9 25.95) (width 0.5) (layer F.Cu) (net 2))
 (segment (start 87.75 23) (end 87.9 23.15) (width 0.5) (layer F.Cu) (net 2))
 (segment (start 87.9 23.15) (end 87.9 25.95) (width 0.5) (layer F.Cu) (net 2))
 (segment (start 77.75 23) (end 77.9 23.15) (width 0.5) (layer F.Cu) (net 2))
 (segment (start 77.9 23.15) (end 77.9 25.95) (width 0.5) (layer F.Cu) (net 2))
 (segment (start 67.75 23) (end 67.9 23.15) (width 0.5) (layer F.Cu) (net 2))
 (segment (start 67.9 23.15) (end 67.9 25.95) (width 0.5) (layer F.Cu) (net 2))
 (segment (start 57.75 23) (end 57.9 23.15) (width 0.5) (layer F.Cu) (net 2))
 (segment (start 57.9 23.15) (end 57.9 25.95) (width 0.5) (layer F.Cu) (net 2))
 (segment (start 47.75 23) (end 47.9 23.15) (width 0.5) (layer F.Cu) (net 2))
 (segment (start 47.9 23.15) (end 47.9 25.95) (width 0.5) (layer F.Cu) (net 2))
 (segment (start 37.75 23) (end 37.9 23.15) (width 0.5) (layer F.Cu) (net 2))
 (segment (start 37.9 23.15) (end 37.9 25.95) (width 0.5) (layer F.Cu) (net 2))
 (segment (start 27.75 23) (end 27.9 23.15) (width 0.5) (layer F.Cu) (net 2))
 (segment (start 27.9 23.15) (end 27.9 25.95) (width 0.5) (layer F.Cu) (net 2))
 (segment (start 27.9 29.05) (end 27.9 32.5) (width 0.5) (layer F.Cu) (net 4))
 (segment (start 27.9 32.5) (end 28 32.5) (width 0.5) (layer F.Cu) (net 4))
 (segment (start 125 25.04) (end 127.04 25.04) (width 0.5) (layer F.Cu) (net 4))
 (segment (start 21.5 29.08) (end 23 27.58) (width 0.5) (layer F.Cu) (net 4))
 (segment (start 21.5 31) (end 21.5 29.08) (width 0.5) (layer F.Cu) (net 4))
 (segment (start 23 32.5) (end 21.5 31) (width 0.5) (layer F.Cu) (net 4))
 (segment (start 126.5 32.5) (end 28 32.5) (width 0.5) (layer F.Cu) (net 4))
 (segment (start 28 32.5) (end 23 32.5) (width 0.5) (layer F.Cu) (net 4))
 (segment (start 128 31) (end 126.5 32.5) (width 0.5) (layer F.Cu) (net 4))
 (segment (start 128 26) (end 128 31) (width 0.5) (layer F.Cu) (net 4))
 (segment (start 127.04 25.04) (end 128 26) (width 0.5) (layer F.Cu) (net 4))
 (segment (start 119 29.05) (end 119 30.5) (width 0.5) (layer F.Cu) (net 5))
 (segment (start 126.58 27.58) (end 125 27.58) (width 0.5) (layer F.Cu) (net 5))
 (segment (start 127 28) (end 126.58 27.58) (width 0.5) (layer F.Cu) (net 5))
 (segment (start 127 30.5) (end 127 28) (width 0.5) (layer F.Cu) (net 5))
 (segment (start 126 31.5) (end 127 30.5) (width 0.5) (layer F.Cu) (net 5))
 (segment (start 120 31.5) (end 126 31.5) (width 0.5) (layer F.Cu) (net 5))
 (segment (start 119 30.5) (end 120 31.5) (width 0.5) (layer F.Cu) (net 5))
 (segment (start 29 29.05) (end 29 30.5) (width 0.5) (layer F.Cu) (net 6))
 (segment (start 37.9 30.6) (end 37.9 29.05) (width 0.5) (layer F.Cu) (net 6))
 (segment (start 37.5 31) (end 37.9 30.6) (width 0.5) (layer F.Cu) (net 6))
 (segment (start 29.5 31) (end 37.5 31) (width 0.5) (layer F.Cu) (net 6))
 (segment (start 29 30.5) (end 29.5 31) (width 0.5) (layer F.Cu) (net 6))
 (segment (start 39 29.05) (end 39 30.5) (width 0.5) (layer F.Cu) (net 7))
 (segment (start 47.9 30.6) (end 47.9 29.05) (width 0.5) (layer F.Cu) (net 7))
 (segment (start 47.5 31) (end 47.9 30.6) (width 0.5) (layer F.Cu) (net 7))
 (segment (start 39.5 31) (end 47.5 31) (width 0.5) (layer F.Cu) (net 7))
 (segment (start 39 30.5) (end 39.5 31) (width 0.5) (layer F.Cu) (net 7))
 (segment (start 49 29.05) (end 49 30.5) (width 0.5) (layer F.Cu) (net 8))
 (segment (start 57.9 30.6) (end 57.9 29.05) (width 0.5) (layer F.Cu) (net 8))
 (segment (start 57.5 31) (end 57.9 30.6) (width 0.5) (layer F.Cu) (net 8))
 (segment (start 49.5 31) (end 57.5 31) (width 0.5) (layer F.Cu) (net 8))
 (segment (start 49 30.5) (end 49.5 31) (width 0.5) (layer F.Cu) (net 8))
 (segment (start 59 29.05) (end 59 30.5) (width 0.5) (layer F.Cu) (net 9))
 (segment (start 67.9 30.6) (end 67.9 29.05) (width 0.5) (layer F.Cu) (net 9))
 (segment (start 67.5 31) (end 67.9 30.6) (width 0.5) (layer F.Cu) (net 9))
 (segment (start 59.5 31) (end 67.5 31) (width 0.5) (layer F.Cu) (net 9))
 (segment (start 59 30.5) (end 59.5 31) (width 0.5) (layer F.Cu) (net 9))
 (segment (start 69 29.05) (end 69 30.5) (width 0.5) (layer F.Cu) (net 10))
 (segment (start 77.9 30.6) (end 77.9 29.05) (width 0.5) (layer F.Cu) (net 10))
 (segment (start 77.5 31) (end 77.9 30.6) (width 0.5) (layer F.Cu) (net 10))
 (segment (start 69.5 31) (end 77.5 31) (width 0.5) (layer F.Cu) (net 10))
 (segment (start 69 30.5) (end 69.5 31) (width 0.5) (layer F.Cu) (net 10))
 (segment (start 79 29.05) (end 79 30.5) (width 0.5) (layer F.Cu) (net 11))
 (segment (start 87.9 30.6) (end 87.9 29.05) (width 0.5) (layer F.Cu) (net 11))
 (segment (start 87.5 31) (end 87.9 30.6) (width 0.5) (layer F.Cu) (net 11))
 (segment (start 79.5 31) (end 87.5 31) (width 0.5) (layer F.Cu) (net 11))
 (segment (start 79 30.5) (end 79.5 31) (width 0.5) (layer F.Cu) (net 11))
 (segment (start 89 29.05) (end 89 30.5) (width 0.5) (layer F.Cu) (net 12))
 (segment (start 97.9 30.6) (end 97.9 29.05) (width 0.5) (layer F.Cu) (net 12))
 (segment (start 97.5 31) (end 97.9 30.6) (width 0.5) (layer F.Cu) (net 12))
 (segment (start 89.5 31) (end 97.5 31) (width 0.5) (layer F.Cu) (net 12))
 (segment (start 89 30.5) (end 89.5 31) (width 0.5) (layer F.Cu) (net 12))
 (segment (start 99 29.05) (end 99 30.5) (width 0.5) (layer F.Cu) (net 13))
 (segment (start 107.9 30.6) (end 107.9 29.05) (width 0.5) (layer F.Cu) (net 13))
 (segment (start 107.5 31) (end 107.9 30.6) (width 0.5) (layer F.Cu) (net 13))
 (segment (start 99.5 31) (end 107.5 31) (width 0.5) (layer F.Cu) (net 13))
 (segment (start 99 30.5) (end 99.5 31) (width 0.5) (layer F.Cu) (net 13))
 (segment (start 109 29.05) (end 109 30.5) (width 0.5) (layer F.Cu) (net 14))
 (segment (start 117.9 30.6) (end 117.9 29.05) (width 0.5) (layer F.Cu) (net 14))
 (segment (start 117.5 31) (end 117.9 30.6) (width 0.5) (layer F.Cu) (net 14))
 (segment (start 109.5 31) (end 117.5 31) (width 0.5) (layer F.Cu) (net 14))
 (segment (start 109 30.5) (end 109.5 31) (width 0.5) (layer F.Cu) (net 14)))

